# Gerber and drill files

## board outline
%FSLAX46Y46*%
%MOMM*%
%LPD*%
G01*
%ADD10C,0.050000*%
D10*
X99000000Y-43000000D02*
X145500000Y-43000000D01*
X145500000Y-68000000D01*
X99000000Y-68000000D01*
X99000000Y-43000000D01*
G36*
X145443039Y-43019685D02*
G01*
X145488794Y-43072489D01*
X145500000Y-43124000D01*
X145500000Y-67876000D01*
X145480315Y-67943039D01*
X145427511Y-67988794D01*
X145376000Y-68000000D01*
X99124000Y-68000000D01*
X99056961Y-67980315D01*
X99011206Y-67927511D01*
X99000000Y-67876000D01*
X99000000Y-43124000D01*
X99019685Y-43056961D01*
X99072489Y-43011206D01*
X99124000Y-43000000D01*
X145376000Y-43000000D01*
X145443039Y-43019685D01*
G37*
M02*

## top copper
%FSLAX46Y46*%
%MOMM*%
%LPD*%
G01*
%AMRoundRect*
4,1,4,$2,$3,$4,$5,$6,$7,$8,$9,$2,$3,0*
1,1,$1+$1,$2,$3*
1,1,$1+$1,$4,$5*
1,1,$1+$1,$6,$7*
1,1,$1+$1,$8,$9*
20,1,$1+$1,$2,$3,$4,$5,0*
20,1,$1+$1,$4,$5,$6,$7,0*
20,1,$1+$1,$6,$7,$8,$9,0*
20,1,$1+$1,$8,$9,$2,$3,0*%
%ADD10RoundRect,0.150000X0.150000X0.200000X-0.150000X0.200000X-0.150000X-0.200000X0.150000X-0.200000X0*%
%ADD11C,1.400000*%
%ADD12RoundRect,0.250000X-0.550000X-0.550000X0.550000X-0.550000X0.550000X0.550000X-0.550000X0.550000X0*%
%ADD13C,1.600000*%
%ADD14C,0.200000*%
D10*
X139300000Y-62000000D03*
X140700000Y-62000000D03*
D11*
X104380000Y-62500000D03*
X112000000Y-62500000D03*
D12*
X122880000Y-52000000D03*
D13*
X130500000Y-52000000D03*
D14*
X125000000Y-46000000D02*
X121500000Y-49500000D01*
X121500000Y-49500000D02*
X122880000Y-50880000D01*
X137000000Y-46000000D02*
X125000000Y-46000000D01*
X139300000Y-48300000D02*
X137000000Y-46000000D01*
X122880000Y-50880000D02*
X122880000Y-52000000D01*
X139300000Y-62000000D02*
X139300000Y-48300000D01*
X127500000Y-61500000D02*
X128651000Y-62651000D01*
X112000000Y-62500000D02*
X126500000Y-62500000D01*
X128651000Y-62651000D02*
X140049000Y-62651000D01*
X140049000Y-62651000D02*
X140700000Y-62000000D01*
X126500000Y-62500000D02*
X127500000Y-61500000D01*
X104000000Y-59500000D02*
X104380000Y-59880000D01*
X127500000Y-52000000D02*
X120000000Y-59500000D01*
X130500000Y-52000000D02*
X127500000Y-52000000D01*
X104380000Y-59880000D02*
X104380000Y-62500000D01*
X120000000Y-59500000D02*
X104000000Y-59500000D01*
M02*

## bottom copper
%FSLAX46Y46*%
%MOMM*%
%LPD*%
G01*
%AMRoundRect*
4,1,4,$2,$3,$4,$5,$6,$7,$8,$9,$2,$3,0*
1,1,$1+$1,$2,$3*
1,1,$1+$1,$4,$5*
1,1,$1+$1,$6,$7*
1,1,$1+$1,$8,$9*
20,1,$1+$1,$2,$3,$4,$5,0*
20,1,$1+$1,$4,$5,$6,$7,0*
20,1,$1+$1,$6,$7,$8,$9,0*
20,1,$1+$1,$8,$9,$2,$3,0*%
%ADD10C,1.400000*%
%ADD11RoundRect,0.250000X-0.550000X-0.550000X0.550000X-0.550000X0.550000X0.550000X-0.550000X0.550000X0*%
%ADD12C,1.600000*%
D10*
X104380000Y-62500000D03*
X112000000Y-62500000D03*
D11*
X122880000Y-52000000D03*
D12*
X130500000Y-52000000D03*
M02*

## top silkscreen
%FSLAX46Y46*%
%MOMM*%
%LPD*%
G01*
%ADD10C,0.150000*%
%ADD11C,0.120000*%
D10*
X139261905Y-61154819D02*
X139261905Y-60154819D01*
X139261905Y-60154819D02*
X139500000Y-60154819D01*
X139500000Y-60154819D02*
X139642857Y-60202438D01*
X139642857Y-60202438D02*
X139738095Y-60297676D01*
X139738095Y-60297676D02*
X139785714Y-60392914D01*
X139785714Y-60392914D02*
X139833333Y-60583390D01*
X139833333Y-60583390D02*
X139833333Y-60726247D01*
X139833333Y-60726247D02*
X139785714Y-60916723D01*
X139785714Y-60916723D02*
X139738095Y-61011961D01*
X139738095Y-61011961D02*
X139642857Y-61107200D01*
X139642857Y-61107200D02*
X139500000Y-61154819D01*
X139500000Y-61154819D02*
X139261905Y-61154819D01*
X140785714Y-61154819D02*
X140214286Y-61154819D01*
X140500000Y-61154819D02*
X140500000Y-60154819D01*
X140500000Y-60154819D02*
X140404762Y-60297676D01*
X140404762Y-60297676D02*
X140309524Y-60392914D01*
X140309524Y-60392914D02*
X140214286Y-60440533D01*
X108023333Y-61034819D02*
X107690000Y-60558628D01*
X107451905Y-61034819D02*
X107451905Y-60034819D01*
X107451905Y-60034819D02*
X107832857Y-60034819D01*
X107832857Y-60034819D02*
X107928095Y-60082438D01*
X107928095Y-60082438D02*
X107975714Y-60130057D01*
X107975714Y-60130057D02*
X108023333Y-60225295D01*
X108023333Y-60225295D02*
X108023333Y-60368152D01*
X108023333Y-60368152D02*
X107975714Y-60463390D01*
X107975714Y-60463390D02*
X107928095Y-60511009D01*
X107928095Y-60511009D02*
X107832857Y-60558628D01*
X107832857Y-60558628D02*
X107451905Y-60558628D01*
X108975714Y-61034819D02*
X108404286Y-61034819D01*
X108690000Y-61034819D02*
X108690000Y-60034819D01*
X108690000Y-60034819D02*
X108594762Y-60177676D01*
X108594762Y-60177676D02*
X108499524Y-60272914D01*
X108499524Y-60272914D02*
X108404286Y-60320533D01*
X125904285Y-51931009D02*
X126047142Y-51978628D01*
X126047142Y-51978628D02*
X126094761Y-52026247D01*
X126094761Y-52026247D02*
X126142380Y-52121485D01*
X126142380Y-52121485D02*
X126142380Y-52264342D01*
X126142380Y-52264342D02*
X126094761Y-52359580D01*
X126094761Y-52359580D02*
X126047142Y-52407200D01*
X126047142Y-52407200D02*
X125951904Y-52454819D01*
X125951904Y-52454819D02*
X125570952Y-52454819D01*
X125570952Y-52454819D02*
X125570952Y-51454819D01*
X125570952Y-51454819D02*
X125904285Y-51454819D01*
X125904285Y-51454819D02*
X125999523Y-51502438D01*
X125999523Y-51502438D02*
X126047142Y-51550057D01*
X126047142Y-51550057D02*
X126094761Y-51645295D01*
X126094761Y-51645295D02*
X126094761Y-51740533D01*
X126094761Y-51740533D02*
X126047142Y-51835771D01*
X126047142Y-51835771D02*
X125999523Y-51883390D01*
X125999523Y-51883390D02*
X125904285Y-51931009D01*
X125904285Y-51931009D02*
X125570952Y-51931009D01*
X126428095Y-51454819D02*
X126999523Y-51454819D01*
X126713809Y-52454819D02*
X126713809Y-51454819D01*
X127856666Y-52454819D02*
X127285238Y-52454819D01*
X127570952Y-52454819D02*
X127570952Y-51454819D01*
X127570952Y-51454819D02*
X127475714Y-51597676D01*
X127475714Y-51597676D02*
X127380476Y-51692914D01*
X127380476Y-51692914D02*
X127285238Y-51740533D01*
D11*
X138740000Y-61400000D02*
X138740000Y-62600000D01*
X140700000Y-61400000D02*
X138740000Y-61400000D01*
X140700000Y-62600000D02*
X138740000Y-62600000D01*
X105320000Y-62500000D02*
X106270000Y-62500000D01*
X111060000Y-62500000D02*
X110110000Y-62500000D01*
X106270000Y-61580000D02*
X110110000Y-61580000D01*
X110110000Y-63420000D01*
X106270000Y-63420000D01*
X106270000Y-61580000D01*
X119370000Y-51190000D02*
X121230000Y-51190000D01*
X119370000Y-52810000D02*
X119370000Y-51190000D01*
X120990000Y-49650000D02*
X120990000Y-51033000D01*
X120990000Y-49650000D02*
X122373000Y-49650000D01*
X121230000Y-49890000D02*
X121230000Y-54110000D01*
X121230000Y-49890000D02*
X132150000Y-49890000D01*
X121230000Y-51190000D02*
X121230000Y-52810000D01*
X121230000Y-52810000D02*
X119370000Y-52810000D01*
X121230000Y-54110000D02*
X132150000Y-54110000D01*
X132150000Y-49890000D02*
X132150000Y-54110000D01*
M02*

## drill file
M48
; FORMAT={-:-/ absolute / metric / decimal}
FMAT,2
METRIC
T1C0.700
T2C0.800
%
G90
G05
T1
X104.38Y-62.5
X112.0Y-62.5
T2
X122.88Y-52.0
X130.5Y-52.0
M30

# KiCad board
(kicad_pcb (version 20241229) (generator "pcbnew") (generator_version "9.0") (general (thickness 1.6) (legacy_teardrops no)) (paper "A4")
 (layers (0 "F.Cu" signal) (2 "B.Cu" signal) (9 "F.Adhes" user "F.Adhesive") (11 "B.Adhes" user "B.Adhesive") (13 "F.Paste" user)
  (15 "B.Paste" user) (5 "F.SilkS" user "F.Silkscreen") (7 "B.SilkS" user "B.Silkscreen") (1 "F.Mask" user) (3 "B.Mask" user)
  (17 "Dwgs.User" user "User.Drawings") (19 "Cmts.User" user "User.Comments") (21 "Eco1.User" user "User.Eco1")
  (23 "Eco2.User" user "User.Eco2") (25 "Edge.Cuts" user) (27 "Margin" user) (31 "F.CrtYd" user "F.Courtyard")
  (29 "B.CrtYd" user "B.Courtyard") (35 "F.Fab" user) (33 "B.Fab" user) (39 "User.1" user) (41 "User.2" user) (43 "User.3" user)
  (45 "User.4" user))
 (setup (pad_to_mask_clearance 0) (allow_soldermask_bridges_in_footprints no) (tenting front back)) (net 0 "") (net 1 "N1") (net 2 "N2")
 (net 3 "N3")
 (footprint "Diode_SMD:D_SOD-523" (layer "F.Cu") (at 140 62)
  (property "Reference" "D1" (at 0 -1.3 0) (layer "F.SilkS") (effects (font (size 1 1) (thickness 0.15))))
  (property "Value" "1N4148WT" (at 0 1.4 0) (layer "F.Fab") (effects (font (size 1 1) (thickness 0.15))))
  (fp_line (start -1.26 -0.6) (end -1.26 0.6) (stroke (width 0.12) (type solid)) (layer "F.SilkS"))
  (fp_line (start 0.7 -0.6) (end -1.26 -0.6) (stroke (width 0.12) (type solid)) (layer "F.SilkS"))
  (fp_line (start 0.7 0.6) (end -1.26 0.6) (stroke (width 0.12) (type solid)) (layer "F.SilkS"))
  (pad "1" smd roundrect (at -0.7 0 180) (size 0.6 0.7) (layers "F.Cu" "F.Mask" "F.Paste") (roundrect_rratio 0.25) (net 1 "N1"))
  (pad "2" smd roundrect (at 0.7 0 180) (size 0.6 0.7) (layers "F.Cu" "F.Mask" "F.Paste") (roundrect_rratio 0.25) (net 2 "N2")))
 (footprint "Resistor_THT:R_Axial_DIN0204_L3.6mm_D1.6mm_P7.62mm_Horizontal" (layer "F.Cu") (at 104.38 62.5)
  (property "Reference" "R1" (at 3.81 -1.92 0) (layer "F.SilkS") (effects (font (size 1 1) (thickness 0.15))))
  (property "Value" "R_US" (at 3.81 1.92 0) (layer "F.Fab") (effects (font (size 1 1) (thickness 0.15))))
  (fp_line (start 0.94 0) (end 1.89 0) (stroke (width 0.12) (type solid)) (layer "F.SilkS"))
  (fp_line (start 6.68 0) (end 5.73 0) (stroke (width 0.12) (type solid)) (layer "F.SilkS"))
  (fp_rect (start 1.89 -0.92) (end 5.73 0.92) (stroke (width 0.12) (type solid)) (fill no) (layer "F.SilkS"))
  (pad "1" thru_hole circle (at 0 0) (size 1.4 1.4) (drill 0.7) (layers "*.Cu" "*.Mask") (remove_unused_layers no) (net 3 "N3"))
  (pad "2" thru_hole circle (at 7.62 0) (size 1.4 1.4) (drill 0.7) (layers "*.Cu" "*.Mask") (remove_unused_layers no) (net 2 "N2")))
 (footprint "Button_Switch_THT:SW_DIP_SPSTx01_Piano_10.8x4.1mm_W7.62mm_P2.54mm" (layer "F.Cu") (at 122.88 52)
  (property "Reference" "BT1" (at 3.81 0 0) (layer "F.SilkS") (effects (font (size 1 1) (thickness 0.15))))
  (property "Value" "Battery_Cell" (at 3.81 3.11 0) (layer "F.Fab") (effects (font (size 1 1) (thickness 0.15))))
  (fp_line (start -3.51 -0.81) (end -1.65 -0.81) (stroke (width 0.12) (type solid)) (layer "F.SilkS"))
  (fp_line (start -3.51 0.81) (end -3.51 -0.81) (stroke (width 0.12) (type solid)) (layer "F.SilkS"))
  (fp_line (start -1.89 -2.35) (end -1.89 -0.967) (stroke (width 0.12) (type solid)) (layer "F.SilkS"))
  (fp_line (start -1.89 -2.35) (end -0.507 -2.35) (stroke (width 0.12) (type solid)) (layer "F.SilkS"))
  (fp_line (start -1.65 -2.11) (end -1.65 2.11) (stroke (width 0.12) (type solid)) (layer "F.SilkS"))
  (fp_line (start -1.65 -2.11) (end 9.27 -2.11) (stroke (width 0.12) (type solid)) (layer "F.SilkS"))
  (fp_line (start -1.65 -0.81) (end -1.65 0.81) (stroke (width 0.12) (type solid)) (layer "F.SilkS"))
  (fp_line (start -1.65 0.81) (end -3.51 0.81) (stroke (width 0.12) (type solid)) (layer "F.SilkS"))
  (fp_line (start -1.65 2.11) (end 9.27 2.11) (stroke (width 0.12) (type solid)) (layer "F.SilkS"))
  (fp_line (start 9.27 -2.11) (end 9.27 2.11) (stroke (width 0.12) (type solid)) (layer "F.SilkS"))
  (pad "1" thru_hole roundrect (at 0 0) (size 1.6 1.6) (drill 0.8) (layers "*.Cu" "*.Mask") (remove_unused_layers no)
   (roundrect_rratio 0.15625) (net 1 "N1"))
  (pad "2" thru_hole circle (at 7.62 0) (size 1.6 1.6) (drill 0.8) (layers "*.Cu" "*.Mask") (remove_unused_layers no) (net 3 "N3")))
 (gr_rect (start 99 43) (end 145.5 68) (stroke (width 0.05) (type default)) (fill no) (layer "Edge.Cuts"))
 (segment (start 125 46) (end 121.5 49.5) (width 0.2) (layer "F.Cu") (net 1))
 (segment (start 121.5 49.5) (end 122.88 50.88) (width 0.2) (layer "F.Cu") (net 1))
 (segment (start 137 46) (end 125 46) (width 0.2) (layer "F.Cu") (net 1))
 (segment (start 139.3 48.3) (end 137 46) (width 0.2) (layer "F.Cu") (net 1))
 (segment (start 122.88 50.88) (end 122.88 52) (width 0.2) (layer "F.Cu") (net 1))
 (segment (start 139.3 62) (end 139.3 48.3) (width 0.2) (layer "F.Cu") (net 1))
 (segment (start 127.5 61.5) (end 128.651 62.651) (width 0.2) (layer "F.Cu") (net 2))
 (segment (start 112 62.5) (end 126.5 62.5) (width 0.2) (layer "F.Cu") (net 2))
 (segment (start 128.651 62.651) (end 140.049 62.651) (width 0.2) (layer "F.Cu") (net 2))
 (segment (start 140.049 62.651) (end 140.7 62) (width 0.2) (layer "F.Cu") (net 2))
 (segment (start 126.5 62.5) (end 127.5 61.5) (width 0.2) (layer "F.Cu") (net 2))
 (segment (start 104 59.5) (end 104.38 59.88) (width 0.2) (layer "F.Cu") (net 3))
 (segment (start 127.5 52) (end 120 59.5) (width 0.2) (layer "F.Cu") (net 3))
 (segment (start 130.5 52) (end 127.5 52) (width 0.2) (layer "F.Cu") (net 3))
 (segment (start 104.38 59.88) (end 104.38 62.5) (width 0.2) (layer "F.Cu") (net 3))
 (segment (start 120 59.5) (end 104 59.5) (width 0.2) (layer "F.Cu") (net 3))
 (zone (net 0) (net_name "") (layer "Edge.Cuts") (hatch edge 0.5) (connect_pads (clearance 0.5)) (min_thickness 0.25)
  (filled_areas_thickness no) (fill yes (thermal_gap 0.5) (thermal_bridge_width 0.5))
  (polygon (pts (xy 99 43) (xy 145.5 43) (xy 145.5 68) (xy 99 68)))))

